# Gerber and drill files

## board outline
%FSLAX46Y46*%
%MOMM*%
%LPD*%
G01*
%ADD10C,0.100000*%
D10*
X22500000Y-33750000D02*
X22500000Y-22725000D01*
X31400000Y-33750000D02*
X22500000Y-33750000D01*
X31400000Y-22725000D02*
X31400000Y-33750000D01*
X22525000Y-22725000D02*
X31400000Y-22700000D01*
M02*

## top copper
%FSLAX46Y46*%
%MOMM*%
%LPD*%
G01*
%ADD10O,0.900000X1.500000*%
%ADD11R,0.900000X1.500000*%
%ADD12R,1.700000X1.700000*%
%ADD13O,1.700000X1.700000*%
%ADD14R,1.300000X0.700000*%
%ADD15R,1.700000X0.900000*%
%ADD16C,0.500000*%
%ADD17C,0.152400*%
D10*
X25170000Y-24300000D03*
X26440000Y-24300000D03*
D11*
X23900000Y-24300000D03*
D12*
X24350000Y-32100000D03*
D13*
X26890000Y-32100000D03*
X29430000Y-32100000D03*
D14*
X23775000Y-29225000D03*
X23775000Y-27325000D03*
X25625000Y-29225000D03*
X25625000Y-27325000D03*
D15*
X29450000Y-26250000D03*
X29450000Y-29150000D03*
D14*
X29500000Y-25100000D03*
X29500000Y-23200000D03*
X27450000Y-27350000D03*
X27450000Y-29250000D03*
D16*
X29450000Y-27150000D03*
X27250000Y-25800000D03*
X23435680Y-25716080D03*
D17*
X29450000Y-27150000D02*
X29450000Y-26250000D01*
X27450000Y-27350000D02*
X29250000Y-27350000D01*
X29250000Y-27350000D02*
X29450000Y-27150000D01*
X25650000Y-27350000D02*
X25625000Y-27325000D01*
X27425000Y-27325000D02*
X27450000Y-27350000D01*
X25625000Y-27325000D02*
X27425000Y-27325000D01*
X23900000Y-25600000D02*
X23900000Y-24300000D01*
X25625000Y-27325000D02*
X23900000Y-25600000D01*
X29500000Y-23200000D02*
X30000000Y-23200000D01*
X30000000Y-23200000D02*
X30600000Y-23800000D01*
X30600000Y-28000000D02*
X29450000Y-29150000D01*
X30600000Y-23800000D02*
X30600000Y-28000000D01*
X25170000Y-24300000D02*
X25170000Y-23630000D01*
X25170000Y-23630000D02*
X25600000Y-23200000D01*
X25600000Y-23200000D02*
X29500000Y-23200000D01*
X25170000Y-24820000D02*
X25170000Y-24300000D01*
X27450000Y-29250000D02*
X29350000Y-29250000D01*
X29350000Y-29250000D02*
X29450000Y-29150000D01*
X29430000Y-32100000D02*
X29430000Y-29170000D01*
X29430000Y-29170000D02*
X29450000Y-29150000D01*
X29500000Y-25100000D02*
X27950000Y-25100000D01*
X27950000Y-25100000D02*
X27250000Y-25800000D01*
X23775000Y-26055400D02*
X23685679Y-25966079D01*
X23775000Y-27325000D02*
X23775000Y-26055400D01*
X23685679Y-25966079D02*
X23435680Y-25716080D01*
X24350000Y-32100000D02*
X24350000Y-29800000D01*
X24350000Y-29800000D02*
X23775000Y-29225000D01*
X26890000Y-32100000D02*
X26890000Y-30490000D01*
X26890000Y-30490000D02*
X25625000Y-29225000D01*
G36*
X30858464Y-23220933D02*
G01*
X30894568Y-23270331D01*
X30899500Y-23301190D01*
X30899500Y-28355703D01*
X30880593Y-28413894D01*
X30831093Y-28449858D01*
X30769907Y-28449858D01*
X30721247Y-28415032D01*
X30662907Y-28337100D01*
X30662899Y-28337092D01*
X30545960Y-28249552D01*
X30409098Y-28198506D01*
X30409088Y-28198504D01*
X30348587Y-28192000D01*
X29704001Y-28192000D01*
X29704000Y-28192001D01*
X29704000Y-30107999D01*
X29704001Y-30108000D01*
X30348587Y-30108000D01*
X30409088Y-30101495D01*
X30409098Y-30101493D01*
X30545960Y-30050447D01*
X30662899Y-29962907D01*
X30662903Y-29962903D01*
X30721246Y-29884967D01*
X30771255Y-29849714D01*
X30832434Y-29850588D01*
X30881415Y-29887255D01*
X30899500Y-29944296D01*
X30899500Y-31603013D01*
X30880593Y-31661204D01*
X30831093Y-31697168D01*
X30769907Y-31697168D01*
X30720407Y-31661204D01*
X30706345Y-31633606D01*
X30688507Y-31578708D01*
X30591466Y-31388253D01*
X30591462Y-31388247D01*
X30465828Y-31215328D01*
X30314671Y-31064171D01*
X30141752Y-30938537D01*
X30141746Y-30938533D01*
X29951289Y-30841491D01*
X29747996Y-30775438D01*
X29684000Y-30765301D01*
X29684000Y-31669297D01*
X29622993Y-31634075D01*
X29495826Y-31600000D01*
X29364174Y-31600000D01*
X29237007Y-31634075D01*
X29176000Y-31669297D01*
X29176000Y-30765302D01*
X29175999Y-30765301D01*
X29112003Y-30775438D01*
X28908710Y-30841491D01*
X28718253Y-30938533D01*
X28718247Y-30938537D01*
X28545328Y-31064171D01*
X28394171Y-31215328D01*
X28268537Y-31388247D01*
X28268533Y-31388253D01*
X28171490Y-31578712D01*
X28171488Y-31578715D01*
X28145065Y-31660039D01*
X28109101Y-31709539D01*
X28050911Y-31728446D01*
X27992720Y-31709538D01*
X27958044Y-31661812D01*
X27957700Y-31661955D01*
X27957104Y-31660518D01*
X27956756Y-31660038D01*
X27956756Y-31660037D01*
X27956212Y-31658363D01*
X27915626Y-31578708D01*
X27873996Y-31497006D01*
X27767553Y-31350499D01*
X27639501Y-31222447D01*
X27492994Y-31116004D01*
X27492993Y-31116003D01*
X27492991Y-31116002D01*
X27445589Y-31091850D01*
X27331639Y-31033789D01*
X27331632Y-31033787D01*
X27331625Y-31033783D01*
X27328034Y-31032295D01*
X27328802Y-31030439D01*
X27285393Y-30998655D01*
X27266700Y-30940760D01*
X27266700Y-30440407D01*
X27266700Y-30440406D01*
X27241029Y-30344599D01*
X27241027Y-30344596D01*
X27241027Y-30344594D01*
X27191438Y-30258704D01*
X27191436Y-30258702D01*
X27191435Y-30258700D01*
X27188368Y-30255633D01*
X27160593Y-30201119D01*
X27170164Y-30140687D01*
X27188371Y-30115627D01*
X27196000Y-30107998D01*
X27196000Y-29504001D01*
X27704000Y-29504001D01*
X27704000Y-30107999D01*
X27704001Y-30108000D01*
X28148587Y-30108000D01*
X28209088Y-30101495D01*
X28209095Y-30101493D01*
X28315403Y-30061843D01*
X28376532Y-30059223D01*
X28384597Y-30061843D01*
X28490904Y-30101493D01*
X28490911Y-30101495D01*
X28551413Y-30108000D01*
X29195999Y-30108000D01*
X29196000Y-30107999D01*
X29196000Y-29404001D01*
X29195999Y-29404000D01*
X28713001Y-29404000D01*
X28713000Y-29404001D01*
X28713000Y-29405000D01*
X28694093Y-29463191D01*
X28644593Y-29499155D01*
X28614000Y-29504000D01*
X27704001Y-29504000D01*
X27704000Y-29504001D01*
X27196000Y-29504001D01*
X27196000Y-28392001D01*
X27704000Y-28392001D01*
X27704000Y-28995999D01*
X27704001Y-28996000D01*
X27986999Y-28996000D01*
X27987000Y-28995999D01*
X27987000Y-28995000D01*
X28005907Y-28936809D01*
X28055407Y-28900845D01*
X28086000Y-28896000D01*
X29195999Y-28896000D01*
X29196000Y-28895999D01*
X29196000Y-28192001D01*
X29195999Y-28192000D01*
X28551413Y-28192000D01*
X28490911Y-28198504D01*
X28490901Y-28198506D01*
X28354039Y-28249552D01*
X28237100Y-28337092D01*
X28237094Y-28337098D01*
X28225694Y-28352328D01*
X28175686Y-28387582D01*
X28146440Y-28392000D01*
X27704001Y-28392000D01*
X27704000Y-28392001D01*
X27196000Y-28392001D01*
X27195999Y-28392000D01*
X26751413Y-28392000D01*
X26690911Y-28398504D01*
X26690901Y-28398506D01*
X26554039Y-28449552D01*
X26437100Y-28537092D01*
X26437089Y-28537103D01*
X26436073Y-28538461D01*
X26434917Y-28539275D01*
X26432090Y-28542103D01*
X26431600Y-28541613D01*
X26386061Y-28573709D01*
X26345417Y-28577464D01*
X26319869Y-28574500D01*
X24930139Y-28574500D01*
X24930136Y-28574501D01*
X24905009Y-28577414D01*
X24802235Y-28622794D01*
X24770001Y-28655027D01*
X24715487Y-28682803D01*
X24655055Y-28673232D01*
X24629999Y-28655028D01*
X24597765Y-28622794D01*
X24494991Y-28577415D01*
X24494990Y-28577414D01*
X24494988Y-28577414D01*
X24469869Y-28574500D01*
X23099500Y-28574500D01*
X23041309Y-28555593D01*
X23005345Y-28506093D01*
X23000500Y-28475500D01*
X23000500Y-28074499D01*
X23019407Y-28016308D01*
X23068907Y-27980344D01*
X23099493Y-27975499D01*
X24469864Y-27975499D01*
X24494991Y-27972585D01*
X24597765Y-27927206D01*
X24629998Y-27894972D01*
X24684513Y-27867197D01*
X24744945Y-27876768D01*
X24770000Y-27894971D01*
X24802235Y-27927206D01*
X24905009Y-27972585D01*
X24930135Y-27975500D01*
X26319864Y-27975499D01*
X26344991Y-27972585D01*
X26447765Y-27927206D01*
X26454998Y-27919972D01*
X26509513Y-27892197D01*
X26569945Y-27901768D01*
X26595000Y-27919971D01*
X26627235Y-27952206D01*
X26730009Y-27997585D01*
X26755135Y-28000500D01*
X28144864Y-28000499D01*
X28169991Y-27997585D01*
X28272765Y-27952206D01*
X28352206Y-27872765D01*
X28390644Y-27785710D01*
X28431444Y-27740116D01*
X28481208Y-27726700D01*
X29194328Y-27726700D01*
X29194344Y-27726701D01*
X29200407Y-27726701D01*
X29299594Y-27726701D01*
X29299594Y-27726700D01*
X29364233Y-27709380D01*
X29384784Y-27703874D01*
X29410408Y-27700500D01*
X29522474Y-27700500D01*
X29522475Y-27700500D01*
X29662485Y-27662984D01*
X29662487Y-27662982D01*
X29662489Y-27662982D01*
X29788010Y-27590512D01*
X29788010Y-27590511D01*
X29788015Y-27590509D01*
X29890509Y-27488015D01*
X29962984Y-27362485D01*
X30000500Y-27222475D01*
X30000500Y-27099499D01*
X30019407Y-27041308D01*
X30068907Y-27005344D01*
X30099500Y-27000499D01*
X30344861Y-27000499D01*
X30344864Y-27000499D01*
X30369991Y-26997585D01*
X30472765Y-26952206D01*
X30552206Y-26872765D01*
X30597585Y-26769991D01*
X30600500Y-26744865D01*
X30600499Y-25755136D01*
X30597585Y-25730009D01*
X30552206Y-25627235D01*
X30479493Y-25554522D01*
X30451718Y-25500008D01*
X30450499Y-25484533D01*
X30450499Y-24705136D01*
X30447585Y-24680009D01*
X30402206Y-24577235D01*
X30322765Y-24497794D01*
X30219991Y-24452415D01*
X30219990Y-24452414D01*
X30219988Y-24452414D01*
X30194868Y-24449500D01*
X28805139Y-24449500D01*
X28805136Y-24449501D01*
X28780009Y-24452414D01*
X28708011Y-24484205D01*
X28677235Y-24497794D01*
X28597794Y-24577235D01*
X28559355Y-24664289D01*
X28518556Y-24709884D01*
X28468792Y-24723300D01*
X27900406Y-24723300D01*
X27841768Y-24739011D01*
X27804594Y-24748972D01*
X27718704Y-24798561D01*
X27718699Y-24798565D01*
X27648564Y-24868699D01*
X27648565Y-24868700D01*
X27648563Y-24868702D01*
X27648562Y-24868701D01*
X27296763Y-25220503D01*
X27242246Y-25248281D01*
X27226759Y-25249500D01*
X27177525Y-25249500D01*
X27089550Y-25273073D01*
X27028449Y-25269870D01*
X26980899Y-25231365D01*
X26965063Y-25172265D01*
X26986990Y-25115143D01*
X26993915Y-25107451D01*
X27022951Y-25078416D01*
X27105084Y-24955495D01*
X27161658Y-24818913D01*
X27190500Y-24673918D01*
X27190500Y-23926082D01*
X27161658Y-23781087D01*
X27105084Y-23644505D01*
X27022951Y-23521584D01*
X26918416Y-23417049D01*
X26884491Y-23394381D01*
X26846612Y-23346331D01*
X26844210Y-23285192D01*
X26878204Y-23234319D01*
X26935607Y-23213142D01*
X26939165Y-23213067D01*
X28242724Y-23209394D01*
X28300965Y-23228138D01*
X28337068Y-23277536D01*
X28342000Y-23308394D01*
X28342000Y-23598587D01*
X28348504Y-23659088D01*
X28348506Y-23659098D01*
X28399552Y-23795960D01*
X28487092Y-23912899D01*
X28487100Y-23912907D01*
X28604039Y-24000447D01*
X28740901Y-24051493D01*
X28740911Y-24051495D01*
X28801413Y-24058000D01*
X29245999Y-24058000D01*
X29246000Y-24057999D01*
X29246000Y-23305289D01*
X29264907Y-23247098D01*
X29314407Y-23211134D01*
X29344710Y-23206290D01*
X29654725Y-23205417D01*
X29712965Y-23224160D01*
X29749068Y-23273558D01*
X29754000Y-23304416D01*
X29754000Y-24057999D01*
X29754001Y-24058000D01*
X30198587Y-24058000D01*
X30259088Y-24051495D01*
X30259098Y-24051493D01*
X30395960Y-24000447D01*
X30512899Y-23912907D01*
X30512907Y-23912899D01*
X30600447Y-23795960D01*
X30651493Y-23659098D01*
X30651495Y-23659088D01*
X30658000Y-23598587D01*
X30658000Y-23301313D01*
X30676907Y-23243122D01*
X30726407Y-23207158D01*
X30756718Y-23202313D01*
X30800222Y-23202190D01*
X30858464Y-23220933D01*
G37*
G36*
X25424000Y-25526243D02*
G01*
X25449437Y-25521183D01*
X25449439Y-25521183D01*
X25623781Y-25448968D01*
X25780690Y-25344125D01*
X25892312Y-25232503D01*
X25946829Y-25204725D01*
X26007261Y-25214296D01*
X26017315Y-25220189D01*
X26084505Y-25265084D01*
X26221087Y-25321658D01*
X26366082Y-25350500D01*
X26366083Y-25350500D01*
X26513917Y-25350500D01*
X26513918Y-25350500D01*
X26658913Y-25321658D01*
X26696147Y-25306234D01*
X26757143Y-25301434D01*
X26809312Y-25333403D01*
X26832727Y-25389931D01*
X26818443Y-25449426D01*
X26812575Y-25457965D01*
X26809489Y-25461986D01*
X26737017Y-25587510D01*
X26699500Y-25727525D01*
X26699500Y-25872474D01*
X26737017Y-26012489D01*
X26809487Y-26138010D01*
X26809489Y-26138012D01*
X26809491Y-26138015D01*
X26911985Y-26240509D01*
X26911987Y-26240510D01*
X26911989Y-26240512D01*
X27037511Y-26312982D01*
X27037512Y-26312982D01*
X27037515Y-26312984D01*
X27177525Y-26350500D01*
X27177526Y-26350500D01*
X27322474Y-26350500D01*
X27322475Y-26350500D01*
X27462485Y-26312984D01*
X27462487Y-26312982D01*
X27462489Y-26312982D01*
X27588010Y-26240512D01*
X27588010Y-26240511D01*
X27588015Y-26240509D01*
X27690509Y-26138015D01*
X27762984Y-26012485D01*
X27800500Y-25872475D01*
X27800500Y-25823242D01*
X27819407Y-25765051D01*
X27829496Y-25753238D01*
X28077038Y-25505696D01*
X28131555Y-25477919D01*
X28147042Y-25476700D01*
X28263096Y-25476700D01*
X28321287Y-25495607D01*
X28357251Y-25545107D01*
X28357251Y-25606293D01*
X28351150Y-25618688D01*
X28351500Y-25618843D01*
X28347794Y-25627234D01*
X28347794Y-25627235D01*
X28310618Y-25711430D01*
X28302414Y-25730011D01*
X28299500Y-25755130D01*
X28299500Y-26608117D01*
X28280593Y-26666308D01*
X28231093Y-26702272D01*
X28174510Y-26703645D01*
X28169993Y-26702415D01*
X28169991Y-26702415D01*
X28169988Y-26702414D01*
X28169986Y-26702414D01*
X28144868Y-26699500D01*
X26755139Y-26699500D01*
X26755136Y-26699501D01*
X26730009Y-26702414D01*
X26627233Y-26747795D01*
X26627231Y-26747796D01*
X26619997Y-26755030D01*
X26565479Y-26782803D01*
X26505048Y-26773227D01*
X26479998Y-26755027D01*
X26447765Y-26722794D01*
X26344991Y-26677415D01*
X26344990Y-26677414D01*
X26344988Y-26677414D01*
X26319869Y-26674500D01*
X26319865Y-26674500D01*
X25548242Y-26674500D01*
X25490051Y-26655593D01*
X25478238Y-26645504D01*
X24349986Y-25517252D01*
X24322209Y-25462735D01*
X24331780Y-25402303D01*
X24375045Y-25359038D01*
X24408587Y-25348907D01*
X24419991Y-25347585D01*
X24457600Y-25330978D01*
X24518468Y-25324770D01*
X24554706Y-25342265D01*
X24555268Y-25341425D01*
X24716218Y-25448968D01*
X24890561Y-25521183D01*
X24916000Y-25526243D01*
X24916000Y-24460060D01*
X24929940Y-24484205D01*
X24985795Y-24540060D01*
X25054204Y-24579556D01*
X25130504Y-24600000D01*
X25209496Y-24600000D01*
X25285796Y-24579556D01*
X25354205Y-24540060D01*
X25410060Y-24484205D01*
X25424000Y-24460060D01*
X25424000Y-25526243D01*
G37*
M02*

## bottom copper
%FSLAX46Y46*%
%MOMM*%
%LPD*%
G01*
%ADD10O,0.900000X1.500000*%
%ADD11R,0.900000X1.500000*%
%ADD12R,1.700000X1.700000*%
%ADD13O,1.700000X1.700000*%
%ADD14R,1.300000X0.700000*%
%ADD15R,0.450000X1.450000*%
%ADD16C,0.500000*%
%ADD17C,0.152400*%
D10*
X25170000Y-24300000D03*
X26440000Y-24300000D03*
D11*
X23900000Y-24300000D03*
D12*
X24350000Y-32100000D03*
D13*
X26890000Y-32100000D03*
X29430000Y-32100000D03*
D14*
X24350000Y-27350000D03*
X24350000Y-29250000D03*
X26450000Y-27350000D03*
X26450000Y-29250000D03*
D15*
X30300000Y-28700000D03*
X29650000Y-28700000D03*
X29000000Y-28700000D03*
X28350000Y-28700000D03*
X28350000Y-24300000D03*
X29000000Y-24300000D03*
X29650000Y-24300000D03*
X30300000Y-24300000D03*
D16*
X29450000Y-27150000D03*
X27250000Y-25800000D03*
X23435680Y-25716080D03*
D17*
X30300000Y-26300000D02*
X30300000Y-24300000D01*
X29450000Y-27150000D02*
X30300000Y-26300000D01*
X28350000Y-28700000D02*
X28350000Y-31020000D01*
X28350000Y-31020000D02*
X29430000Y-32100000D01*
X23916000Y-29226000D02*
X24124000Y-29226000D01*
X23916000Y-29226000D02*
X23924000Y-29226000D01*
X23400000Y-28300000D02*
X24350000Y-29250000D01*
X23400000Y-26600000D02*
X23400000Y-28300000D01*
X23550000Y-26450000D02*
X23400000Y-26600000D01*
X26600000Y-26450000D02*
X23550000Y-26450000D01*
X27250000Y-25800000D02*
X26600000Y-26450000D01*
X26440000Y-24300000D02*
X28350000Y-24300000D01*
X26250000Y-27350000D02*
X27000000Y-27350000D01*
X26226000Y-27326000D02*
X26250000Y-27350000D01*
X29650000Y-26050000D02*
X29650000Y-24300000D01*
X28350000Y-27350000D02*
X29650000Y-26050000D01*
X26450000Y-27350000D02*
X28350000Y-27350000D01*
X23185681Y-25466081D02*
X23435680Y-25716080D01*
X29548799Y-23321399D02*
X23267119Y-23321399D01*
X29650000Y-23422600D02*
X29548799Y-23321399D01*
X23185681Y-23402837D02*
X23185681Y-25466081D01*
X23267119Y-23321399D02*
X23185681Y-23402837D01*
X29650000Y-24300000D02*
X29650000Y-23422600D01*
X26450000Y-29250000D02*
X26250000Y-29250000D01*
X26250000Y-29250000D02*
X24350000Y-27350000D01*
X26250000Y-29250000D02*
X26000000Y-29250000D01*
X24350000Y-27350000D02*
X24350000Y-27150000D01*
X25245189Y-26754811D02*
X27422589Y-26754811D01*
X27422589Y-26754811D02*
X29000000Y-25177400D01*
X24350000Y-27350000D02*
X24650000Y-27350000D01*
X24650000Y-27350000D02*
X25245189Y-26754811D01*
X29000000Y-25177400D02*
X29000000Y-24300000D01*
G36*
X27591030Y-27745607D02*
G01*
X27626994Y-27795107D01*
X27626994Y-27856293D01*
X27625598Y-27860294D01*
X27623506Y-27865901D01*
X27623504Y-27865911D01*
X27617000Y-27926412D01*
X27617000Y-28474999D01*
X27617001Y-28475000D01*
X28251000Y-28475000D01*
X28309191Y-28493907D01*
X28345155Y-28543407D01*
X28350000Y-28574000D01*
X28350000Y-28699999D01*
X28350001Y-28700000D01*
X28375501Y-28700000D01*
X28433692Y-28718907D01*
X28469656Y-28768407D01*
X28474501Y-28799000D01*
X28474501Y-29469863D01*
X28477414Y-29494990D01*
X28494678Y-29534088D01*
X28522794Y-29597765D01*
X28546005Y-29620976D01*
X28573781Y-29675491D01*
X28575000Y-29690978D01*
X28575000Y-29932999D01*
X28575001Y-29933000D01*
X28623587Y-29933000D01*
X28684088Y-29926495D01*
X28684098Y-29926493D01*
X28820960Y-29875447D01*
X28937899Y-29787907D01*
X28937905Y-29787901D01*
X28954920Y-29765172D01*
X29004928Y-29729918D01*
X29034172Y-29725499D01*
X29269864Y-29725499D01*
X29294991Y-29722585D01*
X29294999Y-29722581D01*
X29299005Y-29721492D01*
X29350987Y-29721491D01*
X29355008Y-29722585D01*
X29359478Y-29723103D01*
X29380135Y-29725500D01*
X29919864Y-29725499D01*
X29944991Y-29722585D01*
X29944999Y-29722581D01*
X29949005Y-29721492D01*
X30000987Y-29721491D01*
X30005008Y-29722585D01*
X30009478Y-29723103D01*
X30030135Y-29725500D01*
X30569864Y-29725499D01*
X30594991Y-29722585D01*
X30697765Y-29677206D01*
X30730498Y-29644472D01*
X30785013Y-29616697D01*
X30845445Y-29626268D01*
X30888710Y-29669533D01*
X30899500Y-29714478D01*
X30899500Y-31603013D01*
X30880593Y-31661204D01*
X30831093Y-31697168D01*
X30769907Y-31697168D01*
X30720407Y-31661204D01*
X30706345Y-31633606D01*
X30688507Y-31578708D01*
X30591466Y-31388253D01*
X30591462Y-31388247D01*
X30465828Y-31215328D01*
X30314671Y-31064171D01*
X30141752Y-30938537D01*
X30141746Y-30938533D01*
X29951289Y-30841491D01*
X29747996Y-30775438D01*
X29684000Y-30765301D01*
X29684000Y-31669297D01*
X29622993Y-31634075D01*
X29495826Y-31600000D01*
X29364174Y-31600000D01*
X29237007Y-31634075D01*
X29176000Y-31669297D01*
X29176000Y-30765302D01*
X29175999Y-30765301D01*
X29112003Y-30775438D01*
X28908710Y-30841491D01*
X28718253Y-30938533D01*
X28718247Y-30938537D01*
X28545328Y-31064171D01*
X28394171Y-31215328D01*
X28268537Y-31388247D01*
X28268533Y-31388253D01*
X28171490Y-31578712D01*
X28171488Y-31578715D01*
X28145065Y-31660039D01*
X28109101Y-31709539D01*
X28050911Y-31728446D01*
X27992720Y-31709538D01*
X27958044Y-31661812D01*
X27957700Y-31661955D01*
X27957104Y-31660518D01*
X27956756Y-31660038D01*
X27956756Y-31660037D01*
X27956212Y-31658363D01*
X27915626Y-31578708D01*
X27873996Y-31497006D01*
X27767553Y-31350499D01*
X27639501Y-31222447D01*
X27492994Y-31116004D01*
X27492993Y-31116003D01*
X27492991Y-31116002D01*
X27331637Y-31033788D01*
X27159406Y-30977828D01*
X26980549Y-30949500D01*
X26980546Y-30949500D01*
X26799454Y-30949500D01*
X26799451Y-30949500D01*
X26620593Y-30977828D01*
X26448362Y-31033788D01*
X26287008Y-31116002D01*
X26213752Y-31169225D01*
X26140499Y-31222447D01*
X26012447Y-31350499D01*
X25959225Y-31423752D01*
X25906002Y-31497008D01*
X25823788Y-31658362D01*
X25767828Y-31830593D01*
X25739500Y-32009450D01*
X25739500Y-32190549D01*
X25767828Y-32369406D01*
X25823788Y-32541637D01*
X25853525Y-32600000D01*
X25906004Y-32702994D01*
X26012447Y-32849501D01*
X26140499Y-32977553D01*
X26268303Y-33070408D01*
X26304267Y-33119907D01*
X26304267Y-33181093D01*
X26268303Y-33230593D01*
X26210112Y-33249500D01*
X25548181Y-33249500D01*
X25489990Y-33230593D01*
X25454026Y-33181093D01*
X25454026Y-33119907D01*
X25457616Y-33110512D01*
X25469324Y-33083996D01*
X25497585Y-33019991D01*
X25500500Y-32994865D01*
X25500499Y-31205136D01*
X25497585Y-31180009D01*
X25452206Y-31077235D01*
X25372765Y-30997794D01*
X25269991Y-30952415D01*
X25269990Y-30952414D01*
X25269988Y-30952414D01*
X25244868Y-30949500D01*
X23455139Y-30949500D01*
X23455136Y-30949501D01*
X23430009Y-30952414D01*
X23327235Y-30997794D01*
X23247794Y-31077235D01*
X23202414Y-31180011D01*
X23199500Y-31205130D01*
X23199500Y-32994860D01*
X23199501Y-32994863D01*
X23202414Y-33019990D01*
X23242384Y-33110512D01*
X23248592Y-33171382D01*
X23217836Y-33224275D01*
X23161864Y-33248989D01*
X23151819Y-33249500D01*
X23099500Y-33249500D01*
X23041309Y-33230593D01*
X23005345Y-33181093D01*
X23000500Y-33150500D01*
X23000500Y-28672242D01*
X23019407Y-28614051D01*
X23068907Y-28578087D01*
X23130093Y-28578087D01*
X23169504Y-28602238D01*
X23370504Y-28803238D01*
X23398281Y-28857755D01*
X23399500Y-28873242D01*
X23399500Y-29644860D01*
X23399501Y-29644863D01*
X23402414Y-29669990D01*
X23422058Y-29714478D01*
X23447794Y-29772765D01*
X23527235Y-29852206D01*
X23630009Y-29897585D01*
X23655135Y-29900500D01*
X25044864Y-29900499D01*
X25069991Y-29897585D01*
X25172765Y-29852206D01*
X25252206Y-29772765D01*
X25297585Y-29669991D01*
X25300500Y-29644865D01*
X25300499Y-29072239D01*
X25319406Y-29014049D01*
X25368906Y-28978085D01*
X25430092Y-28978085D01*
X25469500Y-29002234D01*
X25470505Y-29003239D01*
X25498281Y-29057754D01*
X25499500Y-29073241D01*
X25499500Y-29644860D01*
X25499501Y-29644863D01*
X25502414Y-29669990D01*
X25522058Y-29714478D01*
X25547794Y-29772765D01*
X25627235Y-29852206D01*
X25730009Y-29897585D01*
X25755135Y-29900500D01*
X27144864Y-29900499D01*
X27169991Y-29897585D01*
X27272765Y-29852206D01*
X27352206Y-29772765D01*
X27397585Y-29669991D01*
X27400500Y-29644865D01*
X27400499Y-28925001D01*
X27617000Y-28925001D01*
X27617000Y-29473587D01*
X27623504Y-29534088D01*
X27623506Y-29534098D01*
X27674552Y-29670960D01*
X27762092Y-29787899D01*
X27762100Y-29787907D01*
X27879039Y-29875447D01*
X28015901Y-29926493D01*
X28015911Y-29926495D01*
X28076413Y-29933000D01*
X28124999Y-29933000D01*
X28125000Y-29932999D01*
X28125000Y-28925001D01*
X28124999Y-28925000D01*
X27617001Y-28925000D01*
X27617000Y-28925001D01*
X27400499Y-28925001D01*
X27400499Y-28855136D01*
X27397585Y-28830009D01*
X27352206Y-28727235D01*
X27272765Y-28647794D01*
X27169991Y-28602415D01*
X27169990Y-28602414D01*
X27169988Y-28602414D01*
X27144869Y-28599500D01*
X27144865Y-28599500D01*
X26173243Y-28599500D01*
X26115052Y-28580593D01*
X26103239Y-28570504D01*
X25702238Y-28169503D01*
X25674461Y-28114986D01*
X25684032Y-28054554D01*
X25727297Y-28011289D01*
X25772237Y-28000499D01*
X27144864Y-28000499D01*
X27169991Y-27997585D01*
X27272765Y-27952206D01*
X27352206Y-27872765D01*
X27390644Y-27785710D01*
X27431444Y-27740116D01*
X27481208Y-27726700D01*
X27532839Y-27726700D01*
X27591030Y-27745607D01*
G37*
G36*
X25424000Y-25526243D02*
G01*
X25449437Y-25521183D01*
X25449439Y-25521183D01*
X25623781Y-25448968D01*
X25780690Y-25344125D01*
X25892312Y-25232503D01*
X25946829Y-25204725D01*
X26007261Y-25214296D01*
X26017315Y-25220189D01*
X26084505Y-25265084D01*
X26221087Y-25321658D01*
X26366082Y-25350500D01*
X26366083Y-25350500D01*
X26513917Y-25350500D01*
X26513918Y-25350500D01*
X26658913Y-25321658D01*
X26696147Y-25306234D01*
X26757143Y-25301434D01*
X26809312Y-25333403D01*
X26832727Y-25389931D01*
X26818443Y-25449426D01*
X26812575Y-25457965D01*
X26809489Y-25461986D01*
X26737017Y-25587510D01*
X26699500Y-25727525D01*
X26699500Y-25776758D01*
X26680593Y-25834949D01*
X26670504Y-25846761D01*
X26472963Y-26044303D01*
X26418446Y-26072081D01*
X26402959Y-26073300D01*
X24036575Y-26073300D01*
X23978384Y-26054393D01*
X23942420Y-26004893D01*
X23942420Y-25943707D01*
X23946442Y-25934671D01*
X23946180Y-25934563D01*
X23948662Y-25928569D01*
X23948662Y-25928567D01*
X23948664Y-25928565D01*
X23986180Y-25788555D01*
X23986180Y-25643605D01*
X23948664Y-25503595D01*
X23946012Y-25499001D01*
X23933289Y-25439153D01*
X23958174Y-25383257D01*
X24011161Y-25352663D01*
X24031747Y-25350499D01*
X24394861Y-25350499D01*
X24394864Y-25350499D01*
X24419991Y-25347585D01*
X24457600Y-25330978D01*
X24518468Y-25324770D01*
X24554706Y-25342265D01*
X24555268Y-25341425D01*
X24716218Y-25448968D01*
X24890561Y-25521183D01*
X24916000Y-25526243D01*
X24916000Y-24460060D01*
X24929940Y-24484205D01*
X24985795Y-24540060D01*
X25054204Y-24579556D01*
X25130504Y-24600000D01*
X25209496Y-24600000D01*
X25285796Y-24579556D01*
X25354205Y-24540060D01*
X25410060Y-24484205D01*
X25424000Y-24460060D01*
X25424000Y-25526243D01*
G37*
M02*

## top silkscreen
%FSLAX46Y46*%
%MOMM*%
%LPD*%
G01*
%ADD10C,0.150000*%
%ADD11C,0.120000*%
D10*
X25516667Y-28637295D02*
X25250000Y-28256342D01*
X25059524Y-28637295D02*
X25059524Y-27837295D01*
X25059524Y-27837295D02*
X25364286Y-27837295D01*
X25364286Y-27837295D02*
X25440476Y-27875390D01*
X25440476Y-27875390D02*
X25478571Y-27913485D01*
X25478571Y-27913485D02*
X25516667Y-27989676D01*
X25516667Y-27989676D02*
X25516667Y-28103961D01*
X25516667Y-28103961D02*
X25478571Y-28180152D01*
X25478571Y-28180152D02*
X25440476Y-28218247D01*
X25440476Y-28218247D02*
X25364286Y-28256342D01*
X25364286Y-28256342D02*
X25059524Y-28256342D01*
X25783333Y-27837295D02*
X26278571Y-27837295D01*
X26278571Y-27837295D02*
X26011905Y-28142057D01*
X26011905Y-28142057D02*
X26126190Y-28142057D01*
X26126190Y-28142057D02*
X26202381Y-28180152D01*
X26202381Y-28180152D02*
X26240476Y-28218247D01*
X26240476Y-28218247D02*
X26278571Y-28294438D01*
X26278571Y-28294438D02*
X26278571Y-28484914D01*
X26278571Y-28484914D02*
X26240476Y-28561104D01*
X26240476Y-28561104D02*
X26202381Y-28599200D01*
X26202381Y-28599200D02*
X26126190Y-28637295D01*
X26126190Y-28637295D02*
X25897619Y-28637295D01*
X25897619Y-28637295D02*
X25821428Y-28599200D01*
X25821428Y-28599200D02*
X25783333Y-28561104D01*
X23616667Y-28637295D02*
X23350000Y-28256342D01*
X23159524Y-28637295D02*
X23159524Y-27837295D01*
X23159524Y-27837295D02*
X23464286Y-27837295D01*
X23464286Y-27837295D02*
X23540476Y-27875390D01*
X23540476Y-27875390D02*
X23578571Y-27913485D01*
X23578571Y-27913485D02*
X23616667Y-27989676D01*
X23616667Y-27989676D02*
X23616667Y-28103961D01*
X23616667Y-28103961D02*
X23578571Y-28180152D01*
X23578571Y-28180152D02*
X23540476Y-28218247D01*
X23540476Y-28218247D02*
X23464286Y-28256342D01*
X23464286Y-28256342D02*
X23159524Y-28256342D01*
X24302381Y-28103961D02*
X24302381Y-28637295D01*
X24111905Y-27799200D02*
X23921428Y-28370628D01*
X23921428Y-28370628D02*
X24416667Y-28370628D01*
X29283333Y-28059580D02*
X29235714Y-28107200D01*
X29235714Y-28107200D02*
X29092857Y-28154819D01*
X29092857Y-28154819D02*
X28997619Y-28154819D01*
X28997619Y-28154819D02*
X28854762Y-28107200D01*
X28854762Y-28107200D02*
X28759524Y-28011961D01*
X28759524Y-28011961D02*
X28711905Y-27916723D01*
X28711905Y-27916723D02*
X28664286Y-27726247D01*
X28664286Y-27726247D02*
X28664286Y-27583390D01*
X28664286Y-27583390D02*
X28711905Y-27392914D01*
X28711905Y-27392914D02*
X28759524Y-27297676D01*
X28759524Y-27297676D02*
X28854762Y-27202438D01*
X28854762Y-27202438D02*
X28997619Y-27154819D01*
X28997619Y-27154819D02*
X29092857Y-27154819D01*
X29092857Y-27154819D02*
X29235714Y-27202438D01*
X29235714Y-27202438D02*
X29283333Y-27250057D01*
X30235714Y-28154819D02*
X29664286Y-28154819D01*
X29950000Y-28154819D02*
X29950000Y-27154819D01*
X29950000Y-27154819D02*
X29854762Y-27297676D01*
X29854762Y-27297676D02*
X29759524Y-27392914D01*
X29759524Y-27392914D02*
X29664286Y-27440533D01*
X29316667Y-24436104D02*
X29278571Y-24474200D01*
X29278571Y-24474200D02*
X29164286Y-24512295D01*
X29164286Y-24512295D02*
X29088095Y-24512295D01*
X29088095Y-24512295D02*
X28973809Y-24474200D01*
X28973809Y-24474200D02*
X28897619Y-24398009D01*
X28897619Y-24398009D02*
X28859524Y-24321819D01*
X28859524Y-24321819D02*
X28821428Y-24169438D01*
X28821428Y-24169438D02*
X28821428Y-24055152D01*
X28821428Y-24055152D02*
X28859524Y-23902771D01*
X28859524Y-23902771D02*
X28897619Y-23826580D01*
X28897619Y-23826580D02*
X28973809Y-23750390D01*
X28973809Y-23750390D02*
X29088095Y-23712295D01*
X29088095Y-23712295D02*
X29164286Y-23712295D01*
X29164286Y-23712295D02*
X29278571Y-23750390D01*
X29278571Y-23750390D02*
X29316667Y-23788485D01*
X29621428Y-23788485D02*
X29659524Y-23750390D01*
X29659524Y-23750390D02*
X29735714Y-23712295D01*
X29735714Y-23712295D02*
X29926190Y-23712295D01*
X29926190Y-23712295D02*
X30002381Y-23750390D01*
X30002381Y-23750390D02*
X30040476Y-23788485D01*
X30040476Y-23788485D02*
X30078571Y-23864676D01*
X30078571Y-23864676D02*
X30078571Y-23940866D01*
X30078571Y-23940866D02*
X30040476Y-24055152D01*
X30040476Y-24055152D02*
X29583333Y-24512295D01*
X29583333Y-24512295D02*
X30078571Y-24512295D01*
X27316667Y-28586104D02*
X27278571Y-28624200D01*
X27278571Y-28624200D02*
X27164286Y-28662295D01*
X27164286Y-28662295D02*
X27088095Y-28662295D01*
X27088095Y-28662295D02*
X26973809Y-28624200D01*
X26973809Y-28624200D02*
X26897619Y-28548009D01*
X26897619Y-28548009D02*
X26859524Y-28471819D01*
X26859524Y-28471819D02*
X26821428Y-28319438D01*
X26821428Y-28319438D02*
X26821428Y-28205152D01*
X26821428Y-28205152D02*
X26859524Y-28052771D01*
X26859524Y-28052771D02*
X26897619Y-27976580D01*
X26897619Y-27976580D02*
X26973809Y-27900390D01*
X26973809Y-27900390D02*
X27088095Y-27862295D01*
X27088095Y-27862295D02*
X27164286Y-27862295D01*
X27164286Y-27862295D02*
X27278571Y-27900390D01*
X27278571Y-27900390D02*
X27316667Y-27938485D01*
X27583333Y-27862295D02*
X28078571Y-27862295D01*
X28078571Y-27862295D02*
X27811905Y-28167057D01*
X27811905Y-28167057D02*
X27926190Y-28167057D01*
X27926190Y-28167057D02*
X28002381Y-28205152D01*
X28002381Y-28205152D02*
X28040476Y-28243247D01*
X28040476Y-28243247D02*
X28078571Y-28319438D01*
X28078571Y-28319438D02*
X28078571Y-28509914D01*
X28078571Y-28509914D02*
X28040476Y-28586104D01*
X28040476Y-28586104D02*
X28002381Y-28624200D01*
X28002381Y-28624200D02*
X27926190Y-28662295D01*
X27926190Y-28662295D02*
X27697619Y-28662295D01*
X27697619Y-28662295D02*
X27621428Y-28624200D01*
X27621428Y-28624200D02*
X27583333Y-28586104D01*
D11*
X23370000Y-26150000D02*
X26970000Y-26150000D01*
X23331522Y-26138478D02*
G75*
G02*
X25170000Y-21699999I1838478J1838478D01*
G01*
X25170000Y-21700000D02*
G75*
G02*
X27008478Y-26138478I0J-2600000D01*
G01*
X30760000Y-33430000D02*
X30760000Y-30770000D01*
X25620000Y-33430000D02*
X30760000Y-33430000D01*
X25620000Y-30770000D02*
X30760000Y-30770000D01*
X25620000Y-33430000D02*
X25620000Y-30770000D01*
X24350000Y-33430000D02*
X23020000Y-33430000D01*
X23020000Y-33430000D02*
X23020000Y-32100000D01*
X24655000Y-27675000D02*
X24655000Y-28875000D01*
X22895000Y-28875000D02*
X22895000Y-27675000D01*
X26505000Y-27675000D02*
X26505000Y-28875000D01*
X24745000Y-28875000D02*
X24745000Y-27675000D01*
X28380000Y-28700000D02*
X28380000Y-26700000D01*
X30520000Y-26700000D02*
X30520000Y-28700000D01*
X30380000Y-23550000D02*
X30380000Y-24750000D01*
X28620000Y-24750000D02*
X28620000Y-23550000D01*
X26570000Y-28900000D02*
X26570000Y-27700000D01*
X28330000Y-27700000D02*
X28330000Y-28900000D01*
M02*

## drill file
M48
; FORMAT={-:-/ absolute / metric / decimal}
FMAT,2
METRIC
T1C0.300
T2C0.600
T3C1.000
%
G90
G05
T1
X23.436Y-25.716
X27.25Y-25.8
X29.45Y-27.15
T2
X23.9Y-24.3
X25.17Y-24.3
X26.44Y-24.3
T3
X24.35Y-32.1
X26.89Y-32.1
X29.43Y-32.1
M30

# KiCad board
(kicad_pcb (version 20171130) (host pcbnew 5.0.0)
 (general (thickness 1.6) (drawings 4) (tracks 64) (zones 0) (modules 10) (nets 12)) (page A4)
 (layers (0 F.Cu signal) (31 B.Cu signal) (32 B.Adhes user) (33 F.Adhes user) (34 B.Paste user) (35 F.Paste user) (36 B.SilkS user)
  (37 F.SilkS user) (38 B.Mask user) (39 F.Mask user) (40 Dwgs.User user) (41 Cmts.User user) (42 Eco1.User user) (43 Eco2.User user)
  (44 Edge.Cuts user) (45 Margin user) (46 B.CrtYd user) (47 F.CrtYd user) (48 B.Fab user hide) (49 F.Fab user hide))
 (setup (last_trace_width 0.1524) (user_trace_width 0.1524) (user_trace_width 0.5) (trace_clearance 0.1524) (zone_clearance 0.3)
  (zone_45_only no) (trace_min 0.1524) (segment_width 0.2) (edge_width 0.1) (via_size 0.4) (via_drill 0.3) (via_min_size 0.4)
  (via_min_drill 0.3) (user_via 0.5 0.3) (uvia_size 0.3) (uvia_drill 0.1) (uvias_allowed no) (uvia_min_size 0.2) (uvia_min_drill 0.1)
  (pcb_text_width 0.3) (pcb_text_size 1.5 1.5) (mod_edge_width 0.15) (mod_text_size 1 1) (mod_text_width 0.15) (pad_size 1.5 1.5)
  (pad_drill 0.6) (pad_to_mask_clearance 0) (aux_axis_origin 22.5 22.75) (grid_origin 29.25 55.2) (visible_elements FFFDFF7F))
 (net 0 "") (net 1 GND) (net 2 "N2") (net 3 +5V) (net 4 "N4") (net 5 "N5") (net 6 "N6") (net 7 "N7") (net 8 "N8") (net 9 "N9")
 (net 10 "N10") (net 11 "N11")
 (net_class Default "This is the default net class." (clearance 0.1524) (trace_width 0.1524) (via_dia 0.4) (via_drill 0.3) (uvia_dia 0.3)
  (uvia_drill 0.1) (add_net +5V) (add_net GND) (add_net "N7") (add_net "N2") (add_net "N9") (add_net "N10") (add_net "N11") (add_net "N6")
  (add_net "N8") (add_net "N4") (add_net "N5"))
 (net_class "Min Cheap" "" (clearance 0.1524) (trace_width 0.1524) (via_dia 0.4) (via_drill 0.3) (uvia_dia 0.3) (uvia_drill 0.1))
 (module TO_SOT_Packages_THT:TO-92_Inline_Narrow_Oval (layer F.Cu) (at 23.9 24.3)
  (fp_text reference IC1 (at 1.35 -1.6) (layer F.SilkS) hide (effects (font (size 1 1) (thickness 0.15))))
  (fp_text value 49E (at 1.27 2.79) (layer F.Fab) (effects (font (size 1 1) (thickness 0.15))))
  (fp_line (start -0.53 1.85) (end 3.07 1.85) (layer F.SilkS) (width 0.12))
  (fp_arc (start 1.27 0) (end 1.27 -2.6) (angle -135) (layer F.SilkS) (width 0.12))
  (fp_arc (start 1.27 0) (end 1.27 -2.6) (angle 135) (layer F.SilkS) (width 0.12))
  (pad 2 thru_hole oval (at 1.27 0 180) (size 0.9 1.5) (drill 0.6) (layers *.Cu *.Mask) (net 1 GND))
  (pad 3 thru_hole oval (at 2.54 0 180) (size 0.9 1.5) (drill 0.6) (layers *.Cu *.Mask) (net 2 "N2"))
  (pad 1 thru_hole rect (at 0 0 180) (size 0.9 1.5) (drill 0.6) (layers *.Cu *.Mask) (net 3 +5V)))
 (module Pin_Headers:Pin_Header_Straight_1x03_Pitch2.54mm (layer F.Cu) (at 24.35 32.1 90)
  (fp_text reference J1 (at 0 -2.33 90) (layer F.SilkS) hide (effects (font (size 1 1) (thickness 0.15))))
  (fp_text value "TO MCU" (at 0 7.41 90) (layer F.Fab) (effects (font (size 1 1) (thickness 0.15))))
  (fp_line (start -1.33 6.41) (end 1.33 6.41) (layer F.SilkS) (width 0.12))
  (fp_line (start -1.33 1.27) (end -1.33 6.41) (layer F.SilkS) (width 0.12))
  (fp_line (start 1.33 1.27) (end 1.33 6.41) (layer F.SilkS) (width 0.12))
  (fp_line (start -1.33 1.27) (end 1.33 1.27) (layer F.SilkS) (width 0.12))
  (fp_line (start -1.33 0) (end -1.33 -1.33) (layer F.SilkS) (width 0.12))
  (fp_line (start -1.33 -1.33) (end 0 -1.33) (layer F.SilkS) (width 0.12))
  (pad 1 thru_hole rect (at 0 0 90) (size 1.7 1.7) (drill 1) (layers *.Cu *.Mask) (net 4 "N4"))
  (pad 2 thru_hole oval (at 0 2.54 90) (size 1.7 1.7) (drill 1) (layers *.Cu *.Mask) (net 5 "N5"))
  (pad 3 thru_hole oval (at 0 5.08 90) (size 1.7 1.7) (drill 1) (layers *.Cu *.Mask) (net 1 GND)))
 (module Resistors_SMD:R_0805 (layer B.Cu) (at 24.35 28.3 270)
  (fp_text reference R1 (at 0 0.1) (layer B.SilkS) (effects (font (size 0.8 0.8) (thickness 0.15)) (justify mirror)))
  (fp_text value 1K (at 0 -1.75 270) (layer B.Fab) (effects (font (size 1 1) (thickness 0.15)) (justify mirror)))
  (pad 1 smd rect (at -0.95 0 270) (size 0.7 1.3) (layers B.Cu B.Paste B.Mask) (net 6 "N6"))
  (pad 2 smd rect (at 0.95 0 270) (size 0.7 1.3) (layers B.Cu B.Paste B.Mask) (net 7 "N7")))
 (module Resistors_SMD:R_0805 (layer B.Cu) (at 26.45 28.3 270)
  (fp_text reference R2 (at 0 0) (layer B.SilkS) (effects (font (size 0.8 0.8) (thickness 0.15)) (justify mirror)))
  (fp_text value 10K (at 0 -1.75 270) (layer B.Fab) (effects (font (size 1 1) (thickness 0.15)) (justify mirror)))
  (pad 1 smd rect (at -0.95 0 270) (size 0.7 1.3) (layers B.Cu B.Paste B.Mask) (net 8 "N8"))
  (pad 2 smd rect (at 0.95 0 270) (size 0.7 1.3) (layers B.Cu B.Paste B.Mask) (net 6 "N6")))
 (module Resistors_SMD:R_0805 (layer F.Cu) (at 23.775 28.275 90)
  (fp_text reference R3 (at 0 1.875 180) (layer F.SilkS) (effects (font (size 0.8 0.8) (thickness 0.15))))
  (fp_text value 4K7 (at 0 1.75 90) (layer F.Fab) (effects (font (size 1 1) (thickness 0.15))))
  (fp_line (start 0.6 0.88) (end -0.6 0.88) (layer F.SilkS) (width 0.12))
  (fp_line (start -0.6 -0.88) (end 0.6 -0.88) (layer F.SilkS) (width 0.12))
  (pad 1 smd rect (at -0.95 0 90) (size 0.7 1.3) (layers F.Cu F.Paste F.Mask) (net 4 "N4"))
  (pad 2 smd rect (at 0.95 0 90) (size 0.7 1.3) (layers F.Cu F.Paste F.Mask) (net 8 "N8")))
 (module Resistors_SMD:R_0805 (layer F.Cu) (at 25.625 28.275 90)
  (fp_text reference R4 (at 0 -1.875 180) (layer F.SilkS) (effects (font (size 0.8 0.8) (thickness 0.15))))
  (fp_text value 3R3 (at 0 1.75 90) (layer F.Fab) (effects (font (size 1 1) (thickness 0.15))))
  (fp_line (start 0.6 0.88) (end -0.6 0.88) (layer F.SilkS) (width 0.12))
  (fp_line (start -0.6 -0.88) (end 0.6 -0.88) (layer F.SilkS) (width 0.12))
  (pad 1 smd rect (at -0.95 0 90) (size 0.7 1.3) (layers F.Cu F.Paste F.Mask) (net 5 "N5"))
  (pad 2 smd rect (at 0.95 0 90) (size 0.7 1.3) (layers F.Cu F.Paste F.Mask) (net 3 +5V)))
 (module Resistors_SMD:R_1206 (layer F.Cu) (at 29.45 27.7 270)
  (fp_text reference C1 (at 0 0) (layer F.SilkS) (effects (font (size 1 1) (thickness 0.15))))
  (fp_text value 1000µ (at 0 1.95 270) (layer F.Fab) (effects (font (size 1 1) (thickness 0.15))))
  (fp_line (start 1 1.07) (end -1 1.07) (layer F.SilkS) (width 0.12))
  (fp_line (start -1 -1.07) (end 1 -1.07) (layer F.SilkS) (width 0.12))
  (pad 1 smd rect (at -1.45 0 270) (size 0.9 1.7) (layers F.Cu F.Paste F.Mask) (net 3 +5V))
  (pad 2 smd rect (at 1.45 0 270) (size 0.9 1.7) (layers F.Cu F.Paste F.Mask) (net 1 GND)))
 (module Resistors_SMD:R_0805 (layer F.Cu) (at 29.5 24.15 90)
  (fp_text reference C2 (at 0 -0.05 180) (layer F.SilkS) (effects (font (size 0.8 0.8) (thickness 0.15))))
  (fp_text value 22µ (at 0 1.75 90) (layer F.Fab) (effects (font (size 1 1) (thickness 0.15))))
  (fp_line (start 0.6 0.88) (end -0.6 0.88) (layer F.SilkS) (width 0.12))
  (fp_line (start -0.6 -0.88) (end 0.6 -0.88) (layer F.SilkS) (width 0.12))
  (pad 1 smd rect (at -0.95 0 90) (size 0.7 1.3) (layers F.Cu F.Paste F.Mask) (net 7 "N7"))
  (pad 2 smd rect (at 0.95 0 90) (size 0.7 1.3) (layers F.Cu F.Paste F.Mask) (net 1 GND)))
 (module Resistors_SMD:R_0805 (layer F.Cu) (at 27.45 28.3 270)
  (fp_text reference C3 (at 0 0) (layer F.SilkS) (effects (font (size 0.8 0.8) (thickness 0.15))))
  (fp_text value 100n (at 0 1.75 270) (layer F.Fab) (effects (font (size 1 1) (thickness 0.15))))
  (fp_line (start 0.6 0.88) (end -0.6 0.88) (layer F.SilkS) (width 0.12))
  (fp_line (start -0.6 -0.88) (end 0.6 -0.88) (layer F.SilkS) (width 0.12))
  (pad 1 smd rect (at -0.95 0 270) (size 0.7 1.3) (layers F.Cu F.Paste F.Mask) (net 3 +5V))
  (pad 2 smd rect (at 0.95 0 270) (size 0.7 1.3) (layers F.Cu F.Paste F.Mask) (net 1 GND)))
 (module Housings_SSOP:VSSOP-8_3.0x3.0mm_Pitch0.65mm (layer B.Cu) (at 29.325 26.5 90)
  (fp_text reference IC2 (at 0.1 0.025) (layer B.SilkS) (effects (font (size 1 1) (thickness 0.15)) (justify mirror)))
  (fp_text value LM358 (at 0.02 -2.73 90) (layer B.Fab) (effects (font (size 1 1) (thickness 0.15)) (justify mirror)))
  (pad 1 smd rect (at -2.2 0.975 180) (size 0.45 1.45) (layers B.Cu B.Paste B.Mask) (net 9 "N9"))
  (pad 2 smd rect (at -2.2 0.325 180) (size 0.45 1.45) (layers B.Cu B.Paste B.Mask) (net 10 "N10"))
  (pad 3 smd rect (at -2.2 -0.325 180) (size 0.45 1.45) (layers B.Cu B.Paste B.Mask) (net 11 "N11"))
  (pad 4 smd rect (at -2.2 -0.975 180) (size 0.45 1.45) (layers B.Cu B.Paste B.Mask) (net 1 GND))
  (pad 5 smd rect (at 2.2 -0.975 180) (size 0.45 1.45) (layers B.Cu B.Paste B.Mask) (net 2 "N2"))
  (pad 6 smd rect (at 2.2 -0.325 180) (size 0.45 1.45) (layers B.Cu B.Paste B.Mask) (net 6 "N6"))
  (pad 7 smd rect (at 2.2 0.325 180) (size 0.45 1.45) (layers B.Cu B.Paste B.Mask) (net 8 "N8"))
  (pad 8 smd rect (at 2.2 0.975 180) (size 0.45 1.45) (layers B.Cu B.Paste B.Mask) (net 3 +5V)))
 (gr_line (start 22.5 33.75) (end 22.5 22.725) (angle 90) (layer Edge.Cuts) (width 0.1))
 (gr_line (start 31.4 33.75) (end 22.5 33.75) (angle 90) (layer Edge.Cuts) (width 0.1))
 (gr_line (start 31.4 22.725) (end 31.4 33.75) (angle 90) (layer Edge.Cuts) (width 0.1))
 (gr_line (start 22.525 22.725) (end 31.4 22.7) (angle 90) (layer Edge.Cuts) (width 0.1))
 (segment (start 29.45 27.15) (end 29.45 26.25) (width 0.1524) (layer F.Cu) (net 3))
 (segment (start 27.45 27.35) (end 29.25 27.35) (width 0.1524) (layer F.Cu) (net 3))
 (segment (start 30.3 26.3) (end 30.3 24.3) (width 0.1524) (layer B.Cu) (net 3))
 (segment (start 29.45 27.15) (end 30.3 26.3) (width 0.1524) (layer B.Cu) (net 3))
 (via (at 29.45 27.15) (size 0.5) (drill 0.3) (layers F.Cu B.Cu) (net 3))
 (segment (start 29.25 27.35) (end 29.45 27.15) (width 0.1524) (layer F.Cu) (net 3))
 (segment (start 25.65 27.35) (end 25.625 27.325) (width 0.1524) (layer F.Cu) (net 3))
 (segment (start 27.425 27.325) (end 27.45 27.35) (width 0.1524) (layer F.Cu) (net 3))
 (segment (start 25.625 27.325) (end 27.425 27.325) (width 0.1524) (layer F.Cu) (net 3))
 (segment (start 23.9 25.6) (end 23.9 24.3) (width 0.1524) (layer F.Cu) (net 3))
 (segment (start 25.625 27.325) (end 23.9 25.6) (width 0.1524) (layer F.Cu) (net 3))
 (segment (start 29.5 23.2) (end 30 23.2) (width 0.1524) (layer F.Cu) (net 1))
 (segment (start 30 23.2) (end 30.6 23.8) (width 0.1524) (layer F.Cu) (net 1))
 (segment (start 30.6 28) (end 29.45 29.15) (width 0.1524) (layer F.Cu) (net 1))
 (segment (start 30.6 23.8) (end 30.6 28) (width 0.1524) (layer F.Cu) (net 1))
 (segment (start 25.17 24.3) (end 25.17 23.63) (width 0.1524) (layer F.Cu) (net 1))
 (segment (start 25.17 23.63) (end 25.6 23.2) (width 0.1524) (layer F.Cu) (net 1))
 (segment (start 25.6 23.2) (end 29.5 23.2) (width 0.1524) (layer F.Cu) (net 1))
 (segment (start 28.35 28.7) (end 28.35 31.02) (width 0.1524) (layer B.Cu) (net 1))
 (segment (start 28.35 31.02) (end 29.43 32.1) (width 0.1524) (layer B.Cu) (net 1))
 (segment (start 25.17 24.82) (end 25.17 24.3) (width 0.1524) (layer F.Cu) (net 1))
 (segment (start 27.45 29.25) (end 29.35 29.25) (width 0.1524) (layer F.Cu) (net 1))
 (segment (start 29.35 29.25) (end 29.45 29.15) (width 0.1524) (layer F.Cu) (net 1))
 (segment (start 29.43 32.1) (end 29.43 29.17) (width 0.1524) (layer F.Cu) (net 1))
 (segment (start 29.43 29.17) (end 29.45 29.15) (width 0.1524) (layer F.Cu) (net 1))
 (segment (start 29.5 25.1) (end 27.95 25.1) (width 0.1524) (layer F.Cu) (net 7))
 (via (at 27.25 25.8) (size 0.5) (drill 0.3) (layers F.Cu B.Cu) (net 7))
 (segment (start 27.95 25.1) (end 27.25 25.8) (width 0.1524) (layer F.Cu) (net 7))
 (segment (start 23.916 29.226) (end 24.124 29.226) (width 0.1524) (layer B.Cu) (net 7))
 (segment (start 23.916 29.226) (end 23.924 29.226) (width 0.1524) (layer B.Cu) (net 7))
 (segment (start 23.4 28.3) (end 24.35 29.25) (width 0.1524) (layer B.Cu) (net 7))
 (segment (start 23.4 26.6) (end 23.4 28.3) (width 0.1524) (layer B.Cu) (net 7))
 (segment (start 23.55 26.45) (end 23.4 26.6) (width 0.1524) (layer B.Cu) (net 7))
 (segment (start 26.6 26.45) (end 23.55 26.45) (width 0.1524) (layer B.Cu) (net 7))
 (segment (start 27.25 25.8) (end 26.6 26.45) (width 0.1524) (layer B.Cu) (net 7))
 (segment (start 26.44 24.3) (end 28.35 24.3) (width 0.1524) (layer B.Cu) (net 2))
 (segment (start 26.25 27.35) (end 27 27.35) (width 0.1524) (layer B.Cu) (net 8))
 (segment (start 26.226 27.326) (end 26.25 27.35) (width 0.1524) (layer B.Cu) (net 8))
 (segment (start 29.65 26.05) (end 29.65 24.3) (width 0.1524) (layer B.Cu) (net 8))
 (segment (start 28.35 27.35) (end 29.65 26.05) (width 0.1524) (layer B.Cu) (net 8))
 (segment (start 26.45 27.35) (end 28.35 27.35) (width 0.1524) (layer B.Cu) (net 8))
 (via (at 23.43568 25.71608) (size 0.5) (drill 0.3) (layers F.Cu B.Cu) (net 8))
 (segment (start 23.185681 25.466081) (end 23.43568 25.71608) (width 0.1524) (layer B.Cu) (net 8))
 (segment (start 29.548799 23.321399) (end 23.267119 23.321399) (width 0.1524) (layer B.Cu) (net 8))
 (segment (start 29.65 23.4226) (end 29.548799 23.321399) (width 0.1524) (layer B.Cu) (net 8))
 (segment (start 23.775 26.0554) (end 23.685679 25.966079) (width 0.1524) (layer F.Cu) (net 8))
 (segment (start 23.775 27.325) (end 23.775 26.0554) (width 0.1524) (layer F.Cu) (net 8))
 (segment (start 23.685679 25.966079) (end 23.43568 25.71608) (width 0.1524) (layer F.Cu) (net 8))
 (segment (start 23.185681 23.402837) (end 23.185681 25.466081) (width 0.1524) (layer B.Cu) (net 8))
 (segment (start 23.267119 23.321399) (end 23.185681 23.402837) (width 0.1524) (layer B.Cu) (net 8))
 (segment (start 29.65 24.3) (end 29.65 23.4226) (width 0.1524) (layer B.Cu) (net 8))
 (segment (start 26.45 29.25) (end 26.25 29.25) (width 0.1524) (layer B.Cu) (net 6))
 (segment (start 26.25 29.25) (end 24.35 27.35) (width 0.1524) (layer B.Cu) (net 6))
 (segment (start 26.25 29.25) (end 26 29.25) (width 0.1524) (layer B.Cu) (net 6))
 (segment (start 24.35 27.35) (end 24.35 27.15) (width 0.1524) (layer B.Cu) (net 6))
 (segment (start 25.245189 26.754811) (end 27.422589 26.754811) (width 0.1524) (layer B.Cu) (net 6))
 (segment (start 27.422589 26.754811) (end 29 25.1774) (width 0.1524) (layer B.Cu) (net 6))
 (segment (start 24.35 27.35) (end 24.65 27.35) (width 0.1524) (layer B.Cu) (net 6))
 (segment (start 24.65 27.35) (end 25.245189 26.754811) (width 0.1524) (layer B.Cu) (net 6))
 (segment (start 29 25.1774) (end 29 24.3) (width 0.1524) (layer B.Cu) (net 6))
 (segment (start 24.35 32.1) (end 24.35 29.8) (width 0.1524) (layer F.Cu) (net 4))
 (segment (start 24.35 29.8) (end 23.775 29.225) (width 0.1524) (layer F.Cu) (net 4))
 (segment (start 26.89 32.1) (end 26.89 30.49) (width 0.1524) (layer F.Cu) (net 5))
 (segment (start 26.89 30.49) (end 25.625 29.225) (width 0.1524) (layer F.Cu) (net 5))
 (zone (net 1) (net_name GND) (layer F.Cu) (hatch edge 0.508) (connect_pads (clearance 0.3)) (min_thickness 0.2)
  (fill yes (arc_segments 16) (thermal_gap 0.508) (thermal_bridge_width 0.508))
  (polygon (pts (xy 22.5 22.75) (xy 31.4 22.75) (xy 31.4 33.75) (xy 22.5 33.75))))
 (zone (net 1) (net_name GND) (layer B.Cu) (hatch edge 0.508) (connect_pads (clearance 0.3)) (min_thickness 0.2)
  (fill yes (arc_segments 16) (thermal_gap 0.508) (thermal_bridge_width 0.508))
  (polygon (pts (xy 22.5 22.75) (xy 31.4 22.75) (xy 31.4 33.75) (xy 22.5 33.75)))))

